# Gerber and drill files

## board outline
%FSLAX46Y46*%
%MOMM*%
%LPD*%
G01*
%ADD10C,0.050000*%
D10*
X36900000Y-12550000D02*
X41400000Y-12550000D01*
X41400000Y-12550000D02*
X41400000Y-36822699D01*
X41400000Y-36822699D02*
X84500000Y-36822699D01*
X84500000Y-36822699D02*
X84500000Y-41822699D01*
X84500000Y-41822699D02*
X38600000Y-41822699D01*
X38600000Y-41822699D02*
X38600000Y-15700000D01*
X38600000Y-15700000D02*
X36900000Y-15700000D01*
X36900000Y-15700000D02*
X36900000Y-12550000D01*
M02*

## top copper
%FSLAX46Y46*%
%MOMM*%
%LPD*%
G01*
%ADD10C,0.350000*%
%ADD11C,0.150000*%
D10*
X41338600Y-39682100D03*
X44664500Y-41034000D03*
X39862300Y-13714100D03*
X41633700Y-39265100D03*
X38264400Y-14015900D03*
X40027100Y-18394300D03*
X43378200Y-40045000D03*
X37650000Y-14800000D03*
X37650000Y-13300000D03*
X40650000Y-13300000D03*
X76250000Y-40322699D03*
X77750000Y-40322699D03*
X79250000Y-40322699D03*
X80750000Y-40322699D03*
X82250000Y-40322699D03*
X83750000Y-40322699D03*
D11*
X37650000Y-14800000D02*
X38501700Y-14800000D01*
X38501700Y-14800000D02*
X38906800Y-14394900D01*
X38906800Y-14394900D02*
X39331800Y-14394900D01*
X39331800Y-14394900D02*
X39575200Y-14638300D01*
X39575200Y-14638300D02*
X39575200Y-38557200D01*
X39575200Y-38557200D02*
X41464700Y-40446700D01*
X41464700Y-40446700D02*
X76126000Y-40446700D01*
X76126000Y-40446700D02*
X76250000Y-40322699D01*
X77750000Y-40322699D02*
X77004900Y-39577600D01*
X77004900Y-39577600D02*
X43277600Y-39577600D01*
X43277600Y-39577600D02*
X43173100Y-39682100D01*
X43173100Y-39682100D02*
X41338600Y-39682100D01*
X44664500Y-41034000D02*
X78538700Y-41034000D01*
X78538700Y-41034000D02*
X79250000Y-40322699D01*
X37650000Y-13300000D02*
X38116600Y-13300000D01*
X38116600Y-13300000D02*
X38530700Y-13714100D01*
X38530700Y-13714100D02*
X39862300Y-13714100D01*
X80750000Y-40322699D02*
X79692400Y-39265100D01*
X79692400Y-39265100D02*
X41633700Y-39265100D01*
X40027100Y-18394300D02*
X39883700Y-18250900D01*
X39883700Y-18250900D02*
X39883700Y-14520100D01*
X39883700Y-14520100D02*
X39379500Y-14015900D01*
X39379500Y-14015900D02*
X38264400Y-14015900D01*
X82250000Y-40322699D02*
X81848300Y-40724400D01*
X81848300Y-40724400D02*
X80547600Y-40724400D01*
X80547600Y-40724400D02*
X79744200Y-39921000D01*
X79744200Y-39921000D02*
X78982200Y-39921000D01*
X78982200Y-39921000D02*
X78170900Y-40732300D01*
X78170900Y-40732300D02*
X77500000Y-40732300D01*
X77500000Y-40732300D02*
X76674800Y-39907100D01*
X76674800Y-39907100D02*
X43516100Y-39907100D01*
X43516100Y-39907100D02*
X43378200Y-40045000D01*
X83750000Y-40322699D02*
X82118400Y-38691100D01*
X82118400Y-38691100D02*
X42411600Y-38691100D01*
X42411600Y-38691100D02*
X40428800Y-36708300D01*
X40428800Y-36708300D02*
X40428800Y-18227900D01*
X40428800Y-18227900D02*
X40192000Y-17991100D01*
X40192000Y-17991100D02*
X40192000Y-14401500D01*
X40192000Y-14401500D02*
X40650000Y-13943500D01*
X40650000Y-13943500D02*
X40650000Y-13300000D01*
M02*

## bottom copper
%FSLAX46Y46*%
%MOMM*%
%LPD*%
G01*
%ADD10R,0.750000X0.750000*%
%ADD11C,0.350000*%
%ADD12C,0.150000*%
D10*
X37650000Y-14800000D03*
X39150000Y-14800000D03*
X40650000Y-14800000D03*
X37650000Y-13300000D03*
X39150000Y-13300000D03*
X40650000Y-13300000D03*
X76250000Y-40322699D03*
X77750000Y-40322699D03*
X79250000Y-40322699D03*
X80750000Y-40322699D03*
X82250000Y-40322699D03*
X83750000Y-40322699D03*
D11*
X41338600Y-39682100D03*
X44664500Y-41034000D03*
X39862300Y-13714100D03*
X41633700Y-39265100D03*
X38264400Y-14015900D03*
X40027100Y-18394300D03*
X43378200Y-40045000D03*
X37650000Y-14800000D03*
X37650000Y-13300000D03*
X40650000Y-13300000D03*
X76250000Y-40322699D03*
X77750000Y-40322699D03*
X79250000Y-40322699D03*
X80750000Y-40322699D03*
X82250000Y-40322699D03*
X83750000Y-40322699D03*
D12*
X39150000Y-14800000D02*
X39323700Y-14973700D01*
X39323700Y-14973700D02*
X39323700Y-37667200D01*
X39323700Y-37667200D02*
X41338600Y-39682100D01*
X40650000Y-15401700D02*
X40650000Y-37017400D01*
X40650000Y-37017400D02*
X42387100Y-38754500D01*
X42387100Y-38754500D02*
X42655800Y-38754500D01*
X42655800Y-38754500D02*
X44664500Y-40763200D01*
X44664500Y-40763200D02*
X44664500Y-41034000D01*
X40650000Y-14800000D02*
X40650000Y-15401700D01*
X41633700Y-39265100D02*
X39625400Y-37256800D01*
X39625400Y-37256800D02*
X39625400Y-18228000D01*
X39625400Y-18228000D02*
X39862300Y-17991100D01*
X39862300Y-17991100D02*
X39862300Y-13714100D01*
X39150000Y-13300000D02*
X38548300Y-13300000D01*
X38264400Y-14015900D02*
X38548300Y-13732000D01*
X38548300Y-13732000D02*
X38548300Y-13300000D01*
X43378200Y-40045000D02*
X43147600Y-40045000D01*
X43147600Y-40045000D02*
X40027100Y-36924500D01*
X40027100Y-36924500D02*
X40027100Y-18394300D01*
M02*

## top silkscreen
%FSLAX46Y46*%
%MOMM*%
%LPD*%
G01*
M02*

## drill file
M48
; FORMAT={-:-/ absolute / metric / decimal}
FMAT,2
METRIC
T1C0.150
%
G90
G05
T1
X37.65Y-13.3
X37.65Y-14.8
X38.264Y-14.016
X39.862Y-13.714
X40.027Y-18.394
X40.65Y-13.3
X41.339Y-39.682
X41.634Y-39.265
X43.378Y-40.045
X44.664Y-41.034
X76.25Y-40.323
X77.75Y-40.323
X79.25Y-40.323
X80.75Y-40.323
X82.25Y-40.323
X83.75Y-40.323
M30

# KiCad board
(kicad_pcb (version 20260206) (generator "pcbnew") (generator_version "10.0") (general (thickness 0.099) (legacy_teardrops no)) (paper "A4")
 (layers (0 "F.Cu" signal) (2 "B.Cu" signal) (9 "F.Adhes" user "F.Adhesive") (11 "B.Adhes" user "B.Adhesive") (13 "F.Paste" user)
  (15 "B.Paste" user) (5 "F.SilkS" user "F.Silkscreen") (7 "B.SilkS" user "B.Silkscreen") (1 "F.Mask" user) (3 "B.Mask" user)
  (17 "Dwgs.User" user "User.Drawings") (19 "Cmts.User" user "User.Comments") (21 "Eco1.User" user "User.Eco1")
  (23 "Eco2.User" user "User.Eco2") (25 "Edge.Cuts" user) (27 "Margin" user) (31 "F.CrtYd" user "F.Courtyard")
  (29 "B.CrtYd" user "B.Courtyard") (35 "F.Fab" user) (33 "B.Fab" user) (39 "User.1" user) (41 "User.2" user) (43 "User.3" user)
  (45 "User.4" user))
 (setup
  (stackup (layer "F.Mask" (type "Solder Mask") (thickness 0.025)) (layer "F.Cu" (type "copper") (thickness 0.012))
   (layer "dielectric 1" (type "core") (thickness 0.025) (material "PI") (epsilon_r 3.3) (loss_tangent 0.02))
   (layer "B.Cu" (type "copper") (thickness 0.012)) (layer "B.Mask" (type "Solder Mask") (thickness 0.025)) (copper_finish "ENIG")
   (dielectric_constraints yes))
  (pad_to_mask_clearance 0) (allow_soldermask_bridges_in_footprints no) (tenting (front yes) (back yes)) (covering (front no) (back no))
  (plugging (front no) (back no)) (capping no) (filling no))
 (gr_line (start 36.900000000000006 12.55) (end 41.400000000000006 12.55) (stroke (width 0.05) (type default)) (layer "Edge.Cuts"))
 (gr_line (start 41.400000000000006 12.55) (end 41.4 36.822698780255195) (stroke (width 0.05) (type default)) (layer "Edge.Cuts"))
 (gr_line (start 41.4 36.822698780255195) (end 84.5 36.822698780255195) (stroke (width 0.05) (type default)) (layer "Edge.Cuts"))
 (gr_line (start 84.5 36.822698780255195) (end 84.5 41.822698780255195) (stroke (width 0.05) (type default)) (layer "Edge.Cuts"))
 (gr_line (start 84.5 41.822698780255195) (end 38.6 41.822698780255195) (stroke (width 0.05) (type default)) (layer "Edge.Cuts"))
 (gr_line (start 38.6 41.822698780255195) (end 38.6 15.7) (stroke (width 0.05) (type default)) (layer "Edge.Cuts"))
 (gr_line (start 38.6 15.7) (end 36.900000000000006 15.7) (stroke (width 0.05) (type default)) (layer "Edge.Cuts"))
 (gr_line (start 36.900000000000006 15.7) (end 36.900000000000006 12.55) (stroke (width 0.05) (type default)) (layer "Edge.Cuts"))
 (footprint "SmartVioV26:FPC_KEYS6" (layer "F.Cu") (at 0 0)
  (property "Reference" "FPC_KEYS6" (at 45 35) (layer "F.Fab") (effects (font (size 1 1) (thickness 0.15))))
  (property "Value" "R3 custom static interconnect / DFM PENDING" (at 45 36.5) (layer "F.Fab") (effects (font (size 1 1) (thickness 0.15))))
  (pad "S1" smd rect (at 37.650000000000006 14.8) (size 0.75 0.75) (layers "B.Cu" "B.Mask") (solder_mask_margin 0.1) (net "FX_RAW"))
  (pad "S2" smd rect (at 39.150000000000006 14.8) (size 0.75 0.75) (layers "B.Cu" "B.Mask") (solder_mask_margin 0.1) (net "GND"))
  (pad "S3" smd rect (at 40.650000000000006 14.8) (size 0.75 0.75) (layers "B.Cu" "B.Mask") (solder_mask_margin 0.1) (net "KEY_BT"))
  (pad "S4" smd rect (at 37.650000000000006 13.3) (size 0.75 0.75) (layers "B.Cu" "B.Mask") (solder_mask_margin 0.1) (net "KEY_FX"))
  (pad "S5" smd rect (at 39.150000000000006 13.3) (size 0.75 0.75) (layers "B.Cu" "B.Mask") (solder_mask_margin 0.1) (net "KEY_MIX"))
  (pad "S6" smd rect (at 40.650000000000006 13.3) (size 0.75 0.75) (layers "B.Cu" "B.Mask") (solder_mask_margin 0.1) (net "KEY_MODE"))
  (pad "T1" smd rect (at 76.25 40.322698780255195) (size 0.75 0.75) (layers "B.Cu" "B.Mask") (solder_mask_margin 0.1) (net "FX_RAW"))
  (pad "T2" smd rect (at 77.75 40.322698780255195) (size 0.75 0.75) (layers "B.Cu" "B.Mask") (solder_mask_margin 0.1) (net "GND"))
  (pad "T3" smd rect (at 79.25 40.322698780255195) (size 0.75 0.75) (layers "B.Cu" "B.Mask") (solder_mask_margin 0.1) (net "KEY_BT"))
  (pad "T4" smd rect (at 80.75 40.322698780255195) (size 0.75 0.75) (layers "B.Cu" "B.Mask") (solder_mask_margin 0.1) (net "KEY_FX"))
  (pad "T5" smd rect (at 82.25 40.322698780255195) (size 0.75 0.75) (layers "B.Cu" "B.Mask") (solder_mask_margin 0.1) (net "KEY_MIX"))
  (pad "T6" smd rect (at 83.75 40.322698780255195) (size 0.75 0.75) (layers "B.Cu" "B.Mask") (solder_mask_margin 0.1) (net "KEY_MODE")))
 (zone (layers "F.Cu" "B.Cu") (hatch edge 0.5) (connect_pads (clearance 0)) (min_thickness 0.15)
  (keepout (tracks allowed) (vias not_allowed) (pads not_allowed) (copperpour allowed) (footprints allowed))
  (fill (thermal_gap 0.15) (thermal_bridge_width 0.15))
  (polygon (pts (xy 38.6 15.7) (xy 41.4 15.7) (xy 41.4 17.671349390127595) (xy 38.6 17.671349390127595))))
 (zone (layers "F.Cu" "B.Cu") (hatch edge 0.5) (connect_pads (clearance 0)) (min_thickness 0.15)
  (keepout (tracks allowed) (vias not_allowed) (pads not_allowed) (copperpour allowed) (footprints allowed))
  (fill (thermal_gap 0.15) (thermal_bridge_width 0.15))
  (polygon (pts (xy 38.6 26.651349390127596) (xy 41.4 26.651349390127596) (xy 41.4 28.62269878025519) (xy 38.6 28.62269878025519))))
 (segment (start 37.650000000000006 14.8) (end 38.5017 14.8) (width 0.15) (layer "F.Cu") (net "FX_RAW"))
 (segment (start 38.5017 14.8) (end 38.9068 14.3949) (width 0.15) (layer "F.Cu") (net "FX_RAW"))
 (segment (start 38.9068 14.3949) (end 39.3318 14.3949) (width 0.15) (layer "F.Cu") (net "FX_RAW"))
 (segment (start 39.3318 14.3949) (end 39.5752 14.6383) (width 0.15) (layer "F.Cu") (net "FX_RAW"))
 (segment (start 39.5752 14.6383) (end 39.5752 38.5572) (width 0.15) (layer "F.Cu") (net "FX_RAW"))
 (segment (start 39.5752 38.5572) (end 41.4647 40.4467) (width 0.15) (layer "F.Cu") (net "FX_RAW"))
 (segment (start 41.4647 40.4467) (end 76.126 40.4467) (width 0.15) (layer "F.Cu") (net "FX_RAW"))
 (segment (start 76.126 40.4467) (end 76.25 40.322698780255195) (width 0.15) (layer "F.Cu") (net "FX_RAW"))
 (segment (start 39.150000000000006 14.8) (end 39.3237 14.9737) (width 0.15) (layer "B.Cu") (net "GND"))
 (segment (start 39.3237 14.9737) (end 39.3237 37.6672) (width 0.15) (layer "B.Cu") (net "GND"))
 (segment (start 39.3237 37.6672) (end 41.3386 39.6821) (width 0.15) (layer "B.Cu") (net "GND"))
 (segment (start 77.75 40.322698780255195) (end 77.0049 39.577600000000004) (width 0.15) (layer "F.Cu") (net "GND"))
 (segment (start 77.0049 39.577600000000004) (end 43.2776 39.577600000000004) (width 0.15) (layer "F.Cu") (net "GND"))
 (segment (start 43.2776 39.577600000000004) (end 43.1731 39.6821) (width 0.15) (layer "F.Cu") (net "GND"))
 (segment (start 43.1731 39.6821) (end 41.3386 39.6821) (width 0.15) (layer "F.Cu") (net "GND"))
 (via (at 41.3386 39.6821) (size 0.35) (drill 0.15) (layers "F.Cu" "B.Cu") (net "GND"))
 (segment (start 44.6645 41.034) (end 78.5387 41.034) (width 0.15) (layer "F.Cu") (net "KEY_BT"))
 (segment (start 78.5387 41.034) (end 79.25 40.322698780255195) (width 0.15) (layer "F.Cu") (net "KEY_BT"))
 (segment (start 40.65 15.4017) (end 40.65 37.0174) (width 0.15) (layer "B.Cu") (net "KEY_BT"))
 (segment (start 40.65 37.0174) (end 42.3871 38.7545) (width 0.15) (layer "B.Cu") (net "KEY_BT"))
 (segment (start 42.3871 38.7545) (end 42.6558 38.7545) (width 0.15) (layer "B.Cu") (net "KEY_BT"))
 (segment (start 42.6558 38.7545) (end 44.6645 40.763200000000005) (width 0.15) (layer "B.Cu") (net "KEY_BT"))
 (segment (start 44.6645 40.763200000000005) (end 44.6645 41.034) (width 0.15) (layer "B.Cu") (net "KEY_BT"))
 (segment (start 40.650000000000006 14.8) (end 40.65 15.4017) (width 0.15) (layer "B.Cu") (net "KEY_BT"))
 (via (at 44.6645 41.034) (size 0.35) (drill 0.15) (layers "F.Cu" "B.Cu") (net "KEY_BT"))
 (segment (start 37.650000000000006 13.3) (end 38.1166 13.3) (width 0.15) (layer "F.Cu") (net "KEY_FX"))
 (segment (start 38.1166 13.3) (end 38.5307 13.7141) (width 0.15) (layer "F.Cu") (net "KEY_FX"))
 (segment (start 38.5307 13.7141) (end 39.8623 13.7141) (width 0.15) (layer "F.Cu") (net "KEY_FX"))
 (segment (start 41.6337 39.265100000000004) (end 39.6254 37.2568) (width 0.15) (layer "B.Cu") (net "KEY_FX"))
 (segment (start 39.6254 37.2568) (end 39.6254 18.228) (width 0.15) (layer "B.Cu") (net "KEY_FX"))
 (segment (start 39.6254 18.228) (end 39.8623 17.9911) (width 0.15) (layer "B.Cu") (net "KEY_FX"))
 (segment (start 39.8623 17.9911) (end 39.8623 13.7141) (width 0.15) (layer "B.Cu") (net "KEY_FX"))
 (segment (start 80.75 40.322698780255195) (end 79.6924 39.265100000000004) (width 0.15) (layer "F.Cu") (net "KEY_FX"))
 (segment (start 79.6924 39.265100000000004) (end 41.6337 39.265100000000004) (width 0.15) (layer "F.Cu") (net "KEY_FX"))
 (via (at 39.8623 13.7141) (size 0.35) (drill 0.15) (layers "F.Cu" "B.Cu") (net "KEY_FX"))
 (via (at 41.6337 39.265100000000004) (size 0.35) (drill 0.15) (layers "F.Cu" "B.Cu") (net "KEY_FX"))
 (segment (start 39.150000000000006 13.3) (end 38.5483 13.3) (width 0.15) (layer "B.Cu") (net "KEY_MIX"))
 (segment (start 38.2644 14.0159) (end 38.5483 13.732) (width 0.15) (layer "B.Cu") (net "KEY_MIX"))
 (segment (start 38.5483 13.732) (end 38.5483 13.3) (width 0.15) (layer "B.Cu") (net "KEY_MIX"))
 (via (at 38.2644 14.0159) (size 0.35) (drill 0.15) (layers "F.Cu" "B.Cu") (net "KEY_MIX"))
 (segment (start 40.0271 18.3943) (end 39.8837 18.2509) (width 0.15) (layer "F.Cu") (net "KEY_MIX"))
 (segment (start 39.8837 18.2509) (end 39.8837 14.5201) (width 0.15) (layer "F.Cu") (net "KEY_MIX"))
 (segment (start 39.8837 14.5201) (end 39.3795 14.0159) (width 0.15) (layer "F.Cu") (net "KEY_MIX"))
 (segment (start 39.3795 14.0159) (end 38.2644 14.0159) (width 0.15) (layer "F.Cu") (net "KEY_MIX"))
 (via (at 40.0271 18.3943) (size 0.35) (drill 0.15) (layers "F.Cu" "B.Cu") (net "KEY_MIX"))
 (segment (start 43.3782 40.045) (end 43.1476 40.045) (width 0.15) (layer "B.Cu") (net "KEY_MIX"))
 (segment (start 43.1476 40.045) (end 40.0271 36.9245) (width 0.15) (layer "B.Cu") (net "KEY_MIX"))
 (segment (start 40.0271 36.9245) (end 40.0271 18.3943) (width 0.15) (layer "B.Cu") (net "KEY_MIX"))
 (via (at 43.3782 40.045) (size 0.35) (drill 0.15) (layers "F.Cu" "B.Cu") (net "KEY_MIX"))
 (segment (start 82.25 40.322698780255195) (end 81.8483 40.7244) (width 0.15) (layer "F.Cu") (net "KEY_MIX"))
 (segment (start 81.8483 40.7244) (end 80.5476 40.7244) (width 0.15) (layer "F.Cu") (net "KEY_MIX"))
 (segment (start 80.5476 40.7244) (end 79.7442 39.921) (width 0.15) (layer "F.Cu") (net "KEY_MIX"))
 (segment (start 79.7442 39.921) (end 78.9822 39.921) (width 0.15) (layer "F.Cu") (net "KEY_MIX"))
 (segment (start 78.9822 39.921) (end 78.1709 40.7323) (width 0.15) (layer "F.Cu") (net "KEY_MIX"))
 (segment (start 78.1709 40.7323) (end 77.5 40.7323) (width 0.15) (layer "F.Cu") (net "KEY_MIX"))
 (segment (start 77.5 40.7323) (end 76.6748 39.9071) (width 0.15) (layer "F.Cu") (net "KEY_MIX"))
 (segment (start 76.6748 39.9071) (end 43.5161 39.9071) (width 0.15) (layer "F.Cu") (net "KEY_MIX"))
 (segment (start 43.5161 39.9071) (end 43.3782 40.045) (width 0.15) (layer "F.Cu") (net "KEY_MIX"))
 (segment (start 83.75 40.322698780255195) (end 82.1184 38.6911) (width 0.15) (layer "F.Cu") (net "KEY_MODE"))
 (segment (start 82.1184 38.6911) (end 42.4116 38.6911) (width 0.15) (layer "F.Cu") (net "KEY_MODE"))
 (segment (start 42.4116 38.6911) (end 40.4288 36.7083) (width 0.15) (layer "F.Cu") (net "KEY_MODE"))
 (segment (start 40.4288 36.7083) (end 40.4288 18.2279) (width 0.15) (layer "F.Cu") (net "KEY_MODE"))
 (segment (start 40.4288 18.2279) (end 40.192 17.9911) (width 0.15) (layer "F.Cu") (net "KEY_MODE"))
 (segment (start 40.192 17.9911) (end 40.192 14.4015) (width 0.15) (layer "F.Cu") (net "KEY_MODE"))
 (segment (start 40.192 14.4015) (end 40.65 13.9435) (width 0.15) (layer "F.Cu") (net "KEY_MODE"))
 (segment (start 40.65 13.9435) (end 40.650000000000006 13.3) (width 0.15) (layer "F.Cu") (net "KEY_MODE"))
 (via (at 37.650000000000006 14.8) (size 0.35) (drill 0.15) (layers "F.Cu" "B.Cu") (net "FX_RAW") (locked yes))
 (via (at 37.650000000000006 13.3) (size 0.35) (drill 0.15) (layers "F.Cu" "B.Cu") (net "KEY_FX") (locked yes))
 (via (at 40.650000000000006 13.3) (size 0.35) (drill 0.15) (layers "F.Cu" "B.Cu") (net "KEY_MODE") (locked yes))
 (via (at 76.25 40.322698780255195) (size 0.35) (drill 0.15) (layers "F.Cu" "B.Cu") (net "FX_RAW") (locked yes))
 (via (at 77.75 40.322698780255195) (size 0.35) (drill 0.15) (layers "F.Cu" "B.Cu") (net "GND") (locked yes))
 (via (at 79.25 40.322698780255195) (size 0.35) (drill 0.15) (layers "F.Cu" "B.Cu") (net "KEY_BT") (locked yes))
 (via (at 80.75 40.322698780255195) (size 0.35) (drill 0.15) (layers "F.Cu" "B.Cu") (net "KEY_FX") (locked yes))
 (via (at 82.25 40.322698780255195) (size 0.35) (drill 0.15) (layers "F.Cu" "B.Cu") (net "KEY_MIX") (locked yes))
 (via (at 83.75 40.322698780255195) (size 0.35) (drill 0.15) (layers "F.Cu" "B.Cu") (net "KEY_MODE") (locked yes)))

